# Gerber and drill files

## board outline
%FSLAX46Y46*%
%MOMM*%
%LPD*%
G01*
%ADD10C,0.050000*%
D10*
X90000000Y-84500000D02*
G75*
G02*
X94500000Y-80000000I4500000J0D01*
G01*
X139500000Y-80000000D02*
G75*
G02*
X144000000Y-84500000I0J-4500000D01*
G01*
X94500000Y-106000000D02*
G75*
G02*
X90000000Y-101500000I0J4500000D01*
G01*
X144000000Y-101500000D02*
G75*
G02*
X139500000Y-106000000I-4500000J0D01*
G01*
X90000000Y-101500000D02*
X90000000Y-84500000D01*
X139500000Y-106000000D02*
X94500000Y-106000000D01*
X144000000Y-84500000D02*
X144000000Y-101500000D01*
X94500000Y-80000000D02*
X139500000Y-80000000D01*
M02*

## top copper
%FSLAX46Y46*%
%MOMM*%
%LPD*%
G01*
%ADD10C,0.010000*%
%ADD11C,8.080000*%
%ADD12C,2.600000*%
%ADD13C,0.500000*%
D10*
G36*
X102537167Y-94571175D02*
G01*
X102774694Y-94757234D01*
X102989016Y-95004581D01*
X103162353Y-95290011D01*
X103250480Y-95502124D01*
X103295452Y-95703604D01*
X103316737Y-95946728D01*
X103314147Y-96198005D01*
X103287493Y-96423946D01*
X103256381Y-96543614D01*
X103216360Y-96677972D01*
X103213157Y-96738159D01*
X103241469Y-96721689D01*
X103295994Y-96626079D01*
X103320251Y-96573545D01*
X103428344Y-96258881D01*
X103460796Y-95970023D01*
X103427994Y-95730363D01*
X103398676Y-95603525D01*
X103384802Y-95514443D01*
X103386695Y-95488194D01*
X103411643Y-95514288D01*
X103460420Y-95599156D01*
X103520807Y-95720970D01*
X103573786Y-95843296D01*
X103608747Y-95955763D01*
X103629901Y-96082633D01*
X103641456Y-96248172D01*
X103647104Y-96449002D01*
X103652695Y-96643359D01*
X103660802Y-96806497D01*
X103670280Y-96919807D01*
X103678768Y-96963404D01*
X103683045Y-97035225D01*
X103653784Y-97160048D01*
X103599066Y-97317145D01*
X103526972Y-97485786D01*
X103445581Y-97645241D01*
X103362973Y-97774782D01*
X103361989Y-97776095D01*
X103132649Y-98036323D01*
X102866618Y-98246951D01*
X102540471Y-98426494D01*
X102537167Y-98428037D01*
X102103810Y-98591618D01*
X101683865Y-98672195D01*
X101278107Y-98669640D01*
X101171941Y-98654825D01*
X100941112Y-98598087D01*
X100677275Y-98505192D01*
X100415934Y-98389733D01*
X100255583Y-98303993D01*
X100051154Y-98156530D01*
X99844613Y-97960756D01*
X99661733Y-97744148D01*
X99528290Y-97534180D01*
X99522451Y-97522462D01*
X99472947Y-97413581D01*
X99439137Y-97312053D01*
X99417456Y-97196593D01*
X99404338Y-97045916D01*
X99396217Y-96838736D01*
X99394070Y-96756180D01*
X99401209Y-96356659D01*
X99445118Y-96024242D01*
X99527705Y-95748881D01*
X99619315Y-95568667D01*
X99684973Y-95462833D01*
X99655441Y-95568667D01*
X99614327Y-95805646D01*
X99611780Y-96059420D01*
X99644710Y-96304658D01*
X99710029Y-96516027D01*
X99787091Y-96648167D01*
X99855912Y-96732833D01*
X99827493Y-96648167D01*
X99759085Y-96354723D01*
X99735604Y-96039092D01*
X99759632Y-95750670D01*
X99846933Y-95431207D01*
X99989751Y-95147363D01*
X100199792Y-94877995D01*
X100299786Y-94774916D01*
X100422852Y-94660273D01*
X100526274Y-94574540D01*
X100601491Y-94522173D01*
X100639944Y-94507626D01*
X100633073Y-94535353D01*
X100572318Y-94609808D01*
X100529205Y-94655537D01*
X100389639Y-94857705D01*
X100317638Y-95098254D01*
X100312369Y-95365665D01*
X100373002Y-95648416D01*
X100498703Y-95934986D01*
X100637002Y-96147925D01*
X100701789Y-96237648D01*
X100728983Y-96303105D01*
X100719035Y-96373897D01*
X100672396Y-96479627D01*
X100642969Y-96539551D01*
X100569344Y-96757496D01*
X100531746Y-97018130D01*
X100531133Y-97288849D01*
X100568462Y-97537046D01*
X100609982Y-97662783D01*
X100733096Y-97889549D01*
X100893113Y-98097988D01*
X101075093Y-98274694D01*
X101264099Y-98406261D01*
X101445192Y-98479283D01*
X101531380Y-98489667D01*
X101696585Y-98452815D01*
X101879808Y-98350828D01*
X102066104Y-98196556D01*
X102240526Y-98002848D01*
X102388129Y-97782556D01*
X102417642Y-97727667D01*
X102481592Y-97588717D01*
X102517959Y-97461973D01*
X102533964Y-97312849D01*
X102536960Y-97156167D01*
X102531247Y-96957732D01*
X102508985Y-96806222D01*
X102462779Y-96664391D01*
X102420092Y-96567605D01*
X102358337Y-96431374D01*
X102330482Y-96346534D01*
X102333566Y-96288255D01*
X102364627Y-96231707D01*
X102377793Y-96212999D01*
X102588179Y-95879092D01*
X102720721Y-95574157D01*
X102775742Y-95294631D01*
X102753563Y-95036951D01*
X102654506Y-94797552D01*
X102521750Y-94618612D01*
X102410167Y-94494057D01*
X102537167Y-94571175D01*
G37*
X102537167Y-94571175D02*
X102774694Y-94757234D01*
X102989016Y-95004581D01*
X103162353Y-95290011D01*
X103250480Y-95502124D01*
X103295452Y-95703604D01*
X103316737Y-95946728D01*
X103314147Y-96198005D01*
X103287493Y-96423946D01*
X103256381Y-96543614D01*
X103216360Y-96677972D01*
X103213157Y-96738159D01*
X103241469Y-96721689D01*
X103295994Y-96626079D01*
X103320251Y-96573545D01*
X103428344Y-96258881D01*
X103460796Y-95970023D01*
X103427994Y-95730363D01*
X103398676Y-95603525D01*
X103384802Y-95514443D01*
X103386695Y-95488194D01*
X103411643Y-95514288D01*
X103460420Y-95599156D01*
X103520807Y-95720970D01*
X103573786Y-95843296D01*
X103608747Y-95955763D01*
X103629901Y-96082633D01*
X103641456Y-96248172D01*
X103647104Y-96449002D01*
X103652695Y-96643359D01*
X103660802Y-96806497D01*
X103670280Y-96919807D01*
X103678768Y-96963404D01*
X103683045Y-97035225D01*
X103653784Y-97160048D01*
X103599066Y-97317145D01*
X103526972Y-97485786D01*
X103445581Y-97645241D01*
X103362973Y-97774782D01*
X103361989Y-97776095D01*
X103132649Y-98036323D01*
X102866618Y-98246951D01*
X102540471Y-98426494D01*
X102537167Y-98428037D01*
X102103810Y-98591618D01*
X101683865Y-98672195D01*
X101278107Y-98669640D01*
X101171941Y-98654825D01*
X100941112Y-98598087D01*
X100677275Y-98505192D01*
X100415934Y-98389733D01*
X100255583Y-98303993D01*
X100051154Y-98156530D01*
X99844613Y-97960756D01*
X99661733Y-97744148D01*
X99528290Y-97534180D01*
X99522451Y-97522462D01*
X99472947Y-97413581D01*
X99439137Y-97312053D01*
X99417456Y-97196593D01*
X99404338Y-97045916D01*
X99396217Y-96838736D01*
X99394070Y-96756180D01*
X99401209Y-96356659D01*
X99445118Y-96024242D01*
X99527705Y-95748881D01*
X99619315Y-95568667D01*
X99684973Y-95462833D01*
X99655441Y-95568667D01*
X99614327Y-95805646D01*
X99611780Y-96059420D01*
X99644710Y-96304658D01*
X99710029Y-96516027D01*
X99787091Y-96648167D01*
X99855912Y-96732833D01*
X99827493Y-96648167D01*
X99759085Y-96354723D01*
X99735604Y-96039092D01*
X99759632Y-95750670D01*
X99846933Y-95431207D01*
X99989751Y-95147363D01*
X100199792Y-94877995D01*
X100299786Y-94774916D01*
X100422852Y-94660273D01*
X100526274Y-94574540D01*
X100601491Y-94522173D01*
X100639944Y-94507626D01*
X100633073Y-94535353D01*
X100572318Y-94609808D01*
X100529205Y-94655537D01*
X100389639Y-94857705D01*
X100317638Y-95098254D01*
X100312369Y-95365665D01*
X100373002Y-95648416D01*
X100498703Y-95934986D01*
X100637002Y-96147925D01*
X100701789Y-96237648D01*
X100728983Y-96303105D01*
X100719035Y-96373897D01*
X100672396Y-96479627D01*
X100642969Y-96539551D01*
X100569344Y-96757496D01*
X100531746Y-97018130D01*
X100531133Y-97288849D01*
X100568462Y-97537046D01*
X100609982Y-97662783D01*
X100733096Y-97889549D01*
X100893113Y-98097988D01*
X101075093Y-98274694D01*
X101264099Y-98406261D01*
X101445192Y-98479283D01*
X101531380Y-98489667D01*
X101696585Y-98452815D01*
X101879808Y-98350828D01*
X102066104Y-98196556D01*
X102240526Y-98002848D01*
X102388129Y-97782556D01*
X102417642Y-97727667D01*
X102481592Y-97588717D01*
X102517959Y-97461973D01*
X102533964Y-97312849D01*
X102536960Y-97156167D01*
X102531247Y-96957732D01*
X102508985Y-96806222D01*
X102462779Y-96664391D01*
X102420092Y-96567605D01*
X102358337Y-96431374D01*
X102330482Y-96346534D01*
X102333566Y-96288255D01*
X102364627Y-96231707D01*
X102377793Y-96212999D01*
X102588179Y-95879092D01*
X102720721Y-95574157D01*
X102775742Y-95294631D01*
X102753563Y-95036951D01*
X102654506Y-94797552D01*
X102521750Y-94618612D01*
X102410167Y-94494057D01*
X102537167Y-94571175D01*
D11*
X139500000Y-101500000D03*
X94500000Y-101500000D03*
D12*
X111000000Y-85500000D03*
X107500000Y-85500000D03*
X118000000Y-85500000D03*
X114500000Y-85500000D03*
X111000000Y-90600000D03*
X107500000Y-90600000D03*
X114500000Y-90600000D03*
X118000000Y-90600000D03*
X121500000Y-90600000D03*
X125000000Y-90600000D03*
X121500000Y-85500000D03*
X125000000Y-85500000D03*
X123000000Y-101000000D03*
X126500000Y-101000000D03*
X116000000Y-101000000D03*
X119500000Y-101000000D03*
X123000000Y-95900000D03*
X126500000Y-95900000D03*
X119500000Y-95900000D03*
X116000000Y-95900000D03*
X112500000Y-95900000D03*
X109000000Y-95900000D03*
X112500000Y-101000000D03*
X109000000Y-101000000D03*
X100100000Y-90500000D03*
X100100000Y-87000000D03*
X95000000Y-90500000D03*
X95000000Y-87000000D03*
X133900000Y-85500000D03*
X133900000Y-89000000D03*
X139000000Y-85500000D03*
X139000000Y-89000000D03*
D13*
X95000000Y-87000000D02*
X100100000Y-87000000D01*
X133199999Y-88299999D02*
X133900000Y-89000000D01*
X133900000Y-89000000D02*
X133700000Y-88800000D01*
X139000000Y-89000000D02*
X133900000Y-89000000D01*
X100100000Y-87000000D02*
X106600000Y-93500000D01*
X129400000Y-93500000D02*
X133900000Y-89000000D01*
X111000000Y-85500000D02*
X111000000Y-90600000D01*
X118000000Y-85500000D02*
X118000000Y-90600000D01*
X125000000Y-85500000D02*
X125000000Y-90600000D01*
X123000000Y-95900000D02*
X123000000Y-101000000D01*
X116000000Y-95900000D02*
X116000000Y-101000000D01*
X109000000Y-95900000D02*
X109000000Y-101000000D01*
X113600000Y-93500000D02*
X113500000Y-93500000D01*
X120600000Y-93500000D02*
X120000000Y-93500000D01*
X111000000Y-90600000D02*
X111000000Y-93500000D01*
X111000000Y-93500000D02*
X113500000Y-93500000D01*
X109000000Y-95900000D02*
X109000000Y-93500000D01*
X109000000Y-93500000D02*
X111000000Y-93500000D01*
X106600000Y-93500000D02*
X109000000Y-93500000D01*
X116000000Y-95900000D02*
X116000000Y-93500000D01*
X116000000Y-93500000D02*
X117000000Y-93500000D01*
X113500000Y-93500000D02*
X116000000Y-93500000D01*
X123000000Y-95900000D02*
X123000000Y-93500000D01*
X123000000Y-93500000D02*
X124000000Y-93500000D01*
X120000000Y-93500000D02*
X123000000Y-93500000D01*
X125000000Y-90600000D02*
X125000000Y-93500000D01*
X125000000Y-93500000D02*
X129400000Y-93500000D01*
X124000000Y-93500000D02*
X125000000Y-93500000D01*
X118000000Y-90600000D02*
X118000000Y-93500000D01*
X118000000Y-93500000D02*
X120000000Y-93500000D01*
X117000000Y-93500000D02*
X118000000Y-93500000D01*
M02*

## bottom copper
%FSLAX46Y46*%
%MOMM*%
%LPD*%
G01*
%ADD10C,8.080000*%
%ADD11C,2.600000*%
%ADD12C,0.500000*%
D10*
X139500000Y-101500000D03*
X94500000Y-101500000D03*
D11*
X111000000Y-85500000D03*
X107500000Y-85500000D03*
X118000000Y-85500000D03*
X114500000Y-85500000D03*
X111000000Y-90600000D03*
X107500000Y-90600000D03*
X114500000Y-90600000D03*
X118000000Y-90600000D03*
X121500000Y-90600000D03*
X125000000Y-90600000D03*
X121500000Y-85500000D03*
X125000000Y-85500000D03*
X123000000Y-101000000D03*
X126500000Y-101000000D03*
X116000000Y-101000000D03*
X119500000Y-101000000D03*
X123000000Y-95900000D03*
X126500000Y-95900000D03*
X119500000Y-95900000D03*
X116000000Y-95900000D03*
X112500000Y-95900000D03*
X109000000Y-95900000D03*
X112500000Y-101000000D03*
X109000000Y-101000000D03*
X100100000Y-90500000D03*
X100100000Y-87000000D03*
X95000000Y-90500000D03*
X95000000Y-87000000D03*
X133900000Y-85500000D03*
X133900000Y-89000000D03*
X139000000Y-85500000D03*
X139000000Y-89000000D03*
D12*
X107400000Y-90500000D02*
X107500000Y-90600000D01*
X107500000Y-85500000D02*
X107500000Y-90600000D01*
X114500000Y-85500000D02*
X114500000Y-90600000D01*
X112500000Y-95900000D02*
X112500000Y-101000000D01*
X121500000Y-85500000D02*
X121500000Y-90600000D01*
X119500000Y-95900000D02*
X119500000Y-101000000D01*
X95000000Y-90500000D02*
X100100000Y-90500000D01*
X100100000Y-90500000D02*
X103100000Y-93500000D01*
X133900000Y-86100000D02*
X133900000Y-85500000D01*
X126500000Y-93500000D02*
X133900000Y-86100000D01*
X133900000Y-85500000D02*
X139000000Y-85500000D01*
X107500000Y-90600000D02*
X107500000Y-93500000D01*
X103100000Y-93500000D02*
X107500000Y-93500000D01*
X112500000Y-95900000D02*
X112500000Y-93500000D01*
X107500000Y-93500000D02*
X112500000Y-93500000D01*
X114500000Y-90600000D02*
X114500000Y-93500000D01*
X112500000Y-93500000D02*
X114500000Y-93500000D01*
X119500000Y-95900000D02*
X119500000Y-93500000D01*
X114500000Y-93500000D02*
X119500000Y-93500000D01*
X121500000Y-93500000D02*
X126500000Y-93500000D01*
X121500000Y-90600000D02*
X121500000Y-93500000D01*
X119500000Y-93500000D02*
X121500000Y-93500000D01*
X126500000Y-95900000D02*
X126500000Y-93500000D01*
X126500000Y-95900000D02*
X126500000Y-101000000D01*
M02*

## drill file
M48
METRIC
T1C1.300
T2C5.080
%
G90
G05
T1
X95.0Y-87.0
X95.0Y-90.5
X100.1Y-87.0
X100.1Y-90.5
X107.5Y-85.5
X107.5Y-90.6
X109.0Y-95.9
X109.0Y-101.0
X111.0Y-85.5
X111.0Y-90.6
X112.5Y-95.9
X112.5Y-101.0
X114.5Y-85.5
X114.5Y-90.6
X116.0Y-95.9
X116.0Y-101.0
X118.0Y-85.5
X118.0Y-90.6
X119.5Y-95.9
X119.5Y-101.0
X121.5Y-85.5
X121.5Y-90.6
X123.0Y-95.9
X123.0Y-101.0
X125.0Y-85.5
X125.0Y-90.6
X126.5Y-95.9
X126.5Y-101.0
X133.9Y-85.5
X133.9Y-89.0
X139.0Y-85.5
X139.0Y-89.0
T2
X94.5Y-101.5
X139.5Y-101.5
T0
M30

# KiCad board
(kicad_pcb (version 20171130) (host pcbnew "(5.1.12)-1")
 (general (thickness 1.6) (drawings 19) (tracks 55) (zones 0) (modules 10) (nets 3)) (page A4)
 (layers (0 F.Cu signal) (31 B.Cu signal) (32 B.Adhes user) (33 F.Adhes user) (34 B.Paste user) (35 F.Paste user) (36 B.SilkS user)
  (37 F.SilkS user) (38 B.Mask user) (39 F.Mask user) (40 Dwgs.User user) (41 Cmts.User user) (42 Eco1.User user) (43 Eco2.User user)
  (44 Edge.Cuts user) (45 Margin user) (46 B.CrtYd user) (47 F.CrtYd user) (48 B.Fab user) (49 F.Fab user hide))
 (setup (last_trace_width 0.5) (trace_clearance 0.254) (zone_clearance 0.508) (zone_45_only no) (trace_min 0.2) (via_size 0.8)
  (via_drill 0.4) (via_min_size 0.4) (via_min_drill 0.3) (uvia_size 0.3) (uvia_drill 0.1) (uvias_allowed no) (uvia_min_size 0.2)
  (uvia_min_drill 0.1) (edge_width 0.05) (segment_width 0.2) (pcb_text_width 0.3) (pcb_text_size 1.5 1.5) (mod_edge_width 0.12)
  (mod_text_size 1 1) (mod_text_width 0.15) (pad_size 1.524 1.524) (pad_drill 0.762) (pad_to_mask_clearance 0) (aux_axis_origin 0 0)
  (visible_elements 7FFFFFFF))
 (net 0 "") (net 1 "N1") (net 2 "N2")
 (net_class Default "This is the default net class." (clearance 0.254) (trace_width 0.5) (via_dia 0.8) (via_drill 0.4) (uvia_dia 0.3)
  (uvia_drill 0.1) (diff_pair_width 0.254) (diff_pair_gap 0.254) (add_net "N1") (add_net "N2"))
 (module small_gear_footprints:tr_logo (layer F.Cu) (at 132 96.5)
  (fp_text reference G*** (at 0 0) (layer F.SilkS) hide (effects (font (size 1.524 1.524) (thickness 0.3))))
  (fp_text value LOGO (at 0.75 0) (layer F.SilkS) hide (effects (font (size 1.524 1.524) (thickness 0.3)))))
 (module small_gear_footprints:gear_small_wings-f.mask (layer F.Cu) (at 101.5 96.5)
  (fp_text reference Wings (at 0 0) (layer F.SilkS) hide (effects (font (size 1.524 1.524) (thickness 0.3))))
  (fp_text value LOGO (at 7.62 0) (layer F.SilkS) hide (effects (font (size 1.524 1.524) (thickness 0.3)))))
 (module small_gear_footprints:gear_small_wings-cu (layer F.Cu) (at 101.5 96.5)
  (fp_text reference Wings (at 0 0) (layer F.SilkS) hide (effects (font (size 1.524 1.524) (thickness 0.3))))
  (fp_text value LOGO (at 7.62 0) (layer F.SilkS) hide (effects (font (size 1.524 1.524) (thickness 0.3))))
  (fp_poly
   (pts (xy 1.037167 -1.928825) (xy 1.274694 -1.742766) (xy 1.489016 -1.495419) (xy 1.662353 -1.209989) (xy 1.75048 -0.997876)
    (xy 1.795452 -0.796396) (xy 1.816737 -0.553272) (xy 1.814147 -0.301995) (xy 1.787493 -0.076054) (xy 1.756381 0.043614)
    (xy 1.71636 0.177972) (xy 1.713157 0.238159) (xy 1.741469 0.221689) (xy 1.795994 0.126079) (xy 1.820251 0.073545)
    (xy 1.928344 -0.241119) (xy 1.960796 -0.529977) (xy 1.927994 -0.769637) (xy 1.898676 -0.896475) (xy 1.884802 -0.985557)
    (xy 1.886695 -1.011806) (xy 1.911643 -0.985712) (xy 1.96042 -0.900844) (xy 2.020807 -0.77903) (xy 2.073786 -0.656704)
    (xy 2.108747 -0.544237) (xy 2.129901 -0.417367) (xy 2.141456 -0.251828) (xy 2.147104 -0.050998) (xy 2.152695 0.143359)
    (xy 2.160802 0.306497) (xy 2.17028 0.419807) (xy 2.178768 0.463404) (xy 2.183045 0.535225) (xy 2.153784 0.660048) (xy 2.099066 0.817145)
    (xy 2.026972 0.985786) (xy 1.945581 1.145241) (xy 1.862973 1.274782) (xy 1.861989 1.276095) (xy 1.632649 1.536323)
    (xy 1.366618 1.746951) (xy 1.040471 1.926494) (xy 1.037167 1.928037) (xy 0.60381 2.091618) (xy 0.183865 2.172195) (xy -0.221893 2.16964)
    (xy -0.328059 2.154825) (xy -0.558888 2.098087) (xy -0.822725 2.005192) (xy -1.084066 1.889733) (xy -1.244417 1.803993)
    (xy -1.448846 1.65653) (xy -1.655387 1.460756) (xy -1.838267 1.244148) (xy -1.97171 1.03418) (xy -1.977549 1.022462)
    (xy -2.027053 0.913581) (xy -2.060863 0.812053) (xy -2.082544 0.696593) (xy -2.095662 0.545916) (xy -2.103783 0.338736)
    (xy -2.10593 0.25618) (xy -2.098791 -0.143341) (xy -2.054882 -0.475758) (xy -1.972295 -0.751119) (xy -1.880685 -0.931333)
    (xy -1.815027 -1.037167) (xy -1.844559 -0.931333) (xy -1.885673 -0.694354) (xy -1.88822 -0.44058) (xy -1.85529 -0.195342)
    (xy -1.789971 0.016027) (xy -1.712909 0.148167) (xy -1.644088 0.232833) (xy -1.672507 0.148167) (xy -1.740915 -0.145277)
    (xy -1.764396 -0.460908) (xy -1.740368 -0.74933) (xy -1.653067 -1.068793) (xy -1.510249 -1.352637) (xy -1.300208 -1.622005)
    (xy -1.200214 -1.725084) (xy -1.077148 -1.839727) (xy -0.973726 -1.92546) (xy -0.898509 -1.977827) (xy -0.860056 -1.992374)
    (xy -0.866927 -1.964647) (xy -0.927682 -1.890192) (xy -0.970795 -1.844463) (xy -1.110361 -1.642295) (xy -1.182362 -1.401746)
    (xy -1.187631 -1.134335) (xy -1.126998 -0.851584) (xy -1.001297 -0.565014) (xy -0.862998 -0.352075) (xy -0.798211 -0.262352)
    (xy -0.771017 -0.196895) (xy -0.780965 -0.126103) (xy -0.827604 -0.020373) (xy -0.857031 0.039551) (xy -0.930656 0.257496)
    (xy -0.968254 0.51813) (xy -0.968867 0.788849) (xy -0.931538 1.037046) (xy -0.890018 1.162783) (xy -0.766904 1.389549)
    (xy -0.606887 1.597988) (xy -0.424907 1.774694) (xy -0.235901 1.906261) (xy -0.054808 1.979283) (xy 0.03138 1.989667)
    (xy 0.196585 1.952815) (xy 0.379808 1.850828) (xy 0.566104 1.696556) (xy 0.740526 1.502848) (xy 0.888129 1.282556)
    (xy 0.917642 1.227667) (xy 0.981592 1.088717) (xy 1.017959 0.961973) (xy 1.033964 0.812849) (xy 1.03696 0.656167) (xy 1.031247 0.457732)
    (xy 1.008985 0.306222) (xy 0.962779 0.164391) (xy 0.920092 0.067605) (xy 0.858337 -0.068626) (xy 0.830482 -0.153466)
    (xy 0.833566 -0.211745) (xy 0.864627 -0.268293) (xy 0.877793 -0.287001) (xy 1.088179 -0.620908) (xy 1.220721 -0.925843)
    (xy 1.275742 -1.205369) (xy 1.253563 -1.463049) (xy 1.154506 -1.702448) (xy 1.02175 -1.881388) (xy 0.910167 -2.005943)
    (xy 1.037167 -1.928825))
   (layer F.Cu) (width 0.01)))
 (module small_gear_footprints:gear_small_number (layer F.Cu) (at 101.5 96.5)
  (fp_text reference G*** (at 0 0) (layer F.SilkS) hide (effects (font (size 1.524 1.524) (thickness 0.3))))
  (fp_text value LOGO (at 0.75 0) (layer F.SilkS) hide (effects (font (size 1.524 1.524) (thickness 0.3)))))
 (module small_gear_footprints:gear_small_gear (layer F.Cu) (at 101.5 96.5)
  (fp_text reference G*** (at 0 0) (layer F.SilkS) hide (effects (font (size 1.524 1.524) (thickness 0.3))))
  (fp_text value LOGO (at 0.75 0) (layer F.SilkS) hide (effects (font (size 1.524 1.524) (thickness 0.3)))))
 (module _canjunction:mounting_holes (layer F.Cu) (at 94.5 101.5)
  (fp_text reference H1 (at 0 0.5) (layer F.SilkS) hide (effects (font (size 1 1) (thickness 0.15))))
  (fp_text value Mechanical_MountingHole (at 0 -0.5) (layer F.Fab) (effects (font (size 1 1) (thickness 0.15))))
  (pad "" thru_hole circle (at 45 0) (size 8.08 8.08) (drill 5.08) (layers *.Cu *.Mask))
  (pad "" thru_hole circle (at 0 0) (size 8.08 8.08) (drill 5.08) (layers *.Cu *.Mask)))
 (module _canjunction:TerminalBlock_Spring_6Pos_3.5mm (layer F.Cu) (at 125 85.5 180)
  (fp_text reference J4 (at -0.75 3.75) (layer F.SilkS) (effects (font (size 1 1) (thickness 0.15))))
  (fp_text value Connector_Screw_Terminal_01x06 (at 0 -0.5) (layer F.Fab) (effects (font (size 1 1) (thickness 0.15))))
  (pad 5 thru_hole circle (at 14 0 180) (size 2.6 2.6) (drill 1.3) (layers *.Cu *.Mask) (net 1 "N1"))
  (pad 6 thru_hole circle (at 17.5 0 180) (size 2.6 2.6) (drill 1.3) (layers *.Cu *.Mask) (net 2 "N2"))
  (pad 3 thru_hole circle (at 7 0 180) (size 2.6 2.6) (drill 1.3) (layers *.Cu *.Mask) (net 1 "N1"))
  (pad 4 thru_hole circle (at 10.5 0 180) (size 2.6 2.6) (drill 1.3) (layers *.Cu *.Mask) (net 2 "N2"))
  (pad 5 thru_hole circle (at 14 -5.1 180) (size 2.6 2.6) (drill 1.3) (layers *.Cu *.Mask) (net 1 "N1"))
  (pad 6 thru_hole circle (at 17.5 -5.1 180) (size 2.6 2.6) (drill 1.3) (layers *.Cu *.Mask) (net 2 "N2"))
  (pad 4 thru_hole circle (at 10.5 -5.1 180) (size 2.6 2.6) (drill 1.3) (layers *.Cu *.Mask) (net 2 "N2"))
  (pad 3 thru_hole circle (at 7 -5.1 180) (size 2.6 2.6) (drill 1.3) (layers *.Cu *.Mask) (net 1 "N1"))
  (pad 2 thru_hole circle (at 3.5 -5.1 180) (size 2.6 2.6) (drill 1.3) (layers *.Cu *.Mask) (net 2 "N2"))
  (pad 1 thru_hole circle (at 0 -5.1 180) (size 2.6 2.6) (drill 1.3) (layers *.Cu *.Mask) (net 1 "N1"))
  (pad 2 thru_hole circle (at 3.5 0 180) (size 2.6 2.6) (drill 1.3) (layers *.Cu *.Mask) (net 2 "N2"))
  (pad 1 thru_hole circle (at 0 0 180) (size 2.6 2.6) (drill 1.3) (layers *.Cu *.Mask) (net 1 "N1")))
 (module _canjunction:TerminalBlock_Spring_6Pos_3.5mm (layer F.Cu) (at 109 101)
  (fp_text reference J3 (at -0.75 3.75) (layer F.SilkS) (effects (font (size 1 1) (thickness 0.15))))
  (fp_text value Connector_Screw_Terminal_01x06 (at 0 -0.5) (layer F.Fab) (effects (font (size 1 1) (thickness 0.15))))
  (pad 5 thru_hole circle (at 14 0) (size 2.6 2.6) (drill 1.3) (layers *.Cu *.Mask) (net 1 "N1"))
  (pad 6 thru_hole circle (at 17.5 0) (size 2.6 2.6) (drill 1.3) (layers *.Cu *.Mask) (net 2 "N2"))
  (pad 3 thru_hole circle (at 7 0) (size 2.6 2.6) (drill 1.3) (layers *.Cu *.Mask) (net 1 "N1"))
  (pad 4 thru_hole circle (at 10.5 0) (size 2.6 2.6) (drill 1.3) (layers *.Cu *.Mask) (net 2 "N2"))
  (pad 5 thru_hole circle (at 14 -5.1) (size 2.6 2.6) (drill 1.3) (layers *.Cu *.Mask) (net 1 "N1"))
  (pad 6 thru_hole circle (at 17.5 -5.1) (size 2.6 2.6) (drill 1.3) (layers *.Cu *.Mask) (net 2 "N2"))
  (pad 4 thru_hole circle (at 10.5 -5.1) (size 2.6 2.6) (drill 1.3) (layers *.Cu *.Mask) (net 2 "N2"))
  (pad 3 thru_hole circle (at 7 -5.1) (size 2.6 2.6) (drill 1.3) (layers *.Cu *.Mask) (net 1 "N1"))
  (pad 2 thru_hole circle (at 3.5 -5.1) (size 2.6 2.6) (drill 1.3) (layers *.Cu *.Mask) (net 2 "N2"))
  (pad 1 thru_hole circle (at 0 -5.1) (size 2.6 2.6) (drill 1.3) (layers *.Cu *.Mask) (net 1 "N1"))
  (pad 2 thru_hole circle (at 3.5 0) (size 2.6 2.6) (drill 1.3) (layers *.Cu *.Mask) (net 2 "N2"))
  (pad 1 thru_hole circle (at 0 0) (size 2.6 2.6) (drill 1.3) (layers *.Cu *.Mask) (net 1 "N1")))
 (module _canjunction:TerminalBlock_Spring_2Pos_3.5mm (layer F.Cu) (at 95 87 270)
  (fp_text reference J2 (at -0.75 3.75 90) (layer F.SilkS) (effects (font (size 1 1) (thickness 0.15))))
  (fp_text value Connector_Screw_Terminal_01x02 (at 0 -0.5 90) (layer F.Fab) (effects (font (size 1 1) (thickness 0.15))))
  (pad 2 thru_hole circle (at 3.5 -5.1 270) (size 2.6 2.6) (drill 1.3) (layers *.Cu *.Mask) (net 2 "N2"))
  (pad 1 thru_hole circle (at 0 -5.1 270) (size 2.6 2.6) (drill 1.3) (layers *.Cu *.Mask) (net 1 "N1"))
  (pad 2 thru_hole circle (at 3.5 0 270) (size 2.6 2.6) (drill 1.3) (layers *.Cu *.Mask) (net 2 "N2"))
  (pad 1 thru_hole circle (at 0 0 270) (size 2.6 2.6) (drill 1.3) (layers *.Cu *.Mask) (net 1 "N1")))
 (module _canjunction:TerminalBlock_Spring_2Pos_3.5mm (layer F.Cu) (at 139 89 90)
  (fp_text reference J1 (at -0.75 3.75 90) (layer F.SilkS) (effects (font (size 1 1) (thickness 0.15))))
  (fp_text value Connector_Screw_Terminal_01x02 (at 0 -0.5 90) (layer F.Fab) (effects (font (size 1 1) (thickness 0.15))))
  (pad 2 thru_hole circle (at 3.5 -5.1 90) (size 2.6 2.6) (drill 1.3) (layers *.Cu *.Mask) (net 2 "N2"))
  (pad 1 thru_hole circle (at 0 -5.1 90) (size 2.6 2.6) (drill 1.3) (layers *.Cu *.Mask) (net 1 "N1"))
  (pad 2 thru_hole circle (at 3.5 0 90) (size 2.6 2.6) (drill 1.3) (layers *.Cu *.Mask) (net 2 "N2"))
  (pad 1 thru_hole circle (at 0 0 90) (size 2.6 2.6) (drill 1.3) (layers *.Cu *.Mask) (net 1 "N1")))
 (gr_arc (start 94.5 84.5) (end 94.5 80) (angle -90) (layer Edge.Cuts) (width 0.05))
 (gr_arc (start 139.5 84.5) (end 144 84.5) (angle -90) (layer Edge.Cuts) (width 0.05))
 (gr_arc (start 94.5 101.5) (end 90 101.5) (angle -90) (layer Edge.Cuts) (width 0.05))
 (gr_arc (start 139.5 101.5) (end 139.5 106) (angle -90) (layer Edge.Cuts) (width 0.05))
 (gr_line (start 90 101.5) (end 90 84.5) (layer Edge.Cuts) (width 0.05))
 (gr_line (start 139.5 106) (end 94.5 106) (layer Edge.Cuts) (width 0.05))
 (gr_line (start 144 84.5) (end 144 101.5) (layer Edge.Cuts) (width 0.05))
 (gr_line (start 94.5 80) (end 139.5 80) (layer Edge.Cuts) (width 0.05))
 (segment (start 107.4 90.5) (end 107.5 90.6) (width 0.5) (layer B.Cu) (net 2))
 (segment (start 107.5 85.5) (end 107.5 90.6) (width 0.5) (layer B.Cu) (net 2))
 (segment (start 114.5 85.5) (end 114.5 90.6) (width 0.5) (layer B.Cu) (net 2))
 (segment (start 112.5 95.9) (end 112.5 101) (width 0.5) (layer B.Cu) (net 2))
 (segment (start 121.5 85.5) (end 121.5 90.6) (width 0.5) (layer B.Cu) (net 2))
 (segment (start 119.5 95.9) (end 119.5 101) (width 0.5) (layer B.Cu) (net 2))
 (segment (start 95 90.5) (end 100.1 90.5) (width 0.5) (layer B.Cu) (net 2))
 (segment (start 100.1 90.5) (end 103.1 93.5) (width 0.5) (layer B.Cu) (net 2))
 (segment (start 133.9 86.1) (end 133.9 85.5) (width 0.5) (layer B.Cu) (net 2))
 (segment (start 126.5 93.5) (end 133.9 86.1) (width 0.5) (layer B.Cu) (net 2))
 (segment (start 133.9 85.5) (end 139 85.5) (width 0.5) (layer B.Cu) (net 2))
 (segment (start 107.5 90.6) (end 107.5 93.5) (width 0.5) (layer B.Cu) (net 2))
 (segment (start 103.1 93.5) (end 107.5 93.5) (width 0.5) (layer B.Cu) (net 2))
 (segment (start 112.5 95.9) (end 112.5 93.5) (width 0.5) (layer B.Cu) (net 2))
 (segment (start 107.5 93.5) (end 112.5 93.5) (width 0.5) (layer B.Cu) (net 2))
 (segment (start 114.5 90.6) (end 114.5 93.5) (width 0.5) (layer B.Cu) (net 2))
 (segment (start 112.5 93.5) (end 114.5 93.5) (width 0.5) (layer B.Cu) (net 2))
 (segment (start 119.5 95.9) (end 119.5 93.5) (width 0.5) (layer B.Cu) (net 2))
 (segment (start 114.5 93.5) (end 119.5 93.5) (width 0.5) (layer B.Cu) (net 2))
 (segment (start 121.5 93.5) (end 126.5 93.5) (width 0.5) (layer B.Cu) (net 2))
 (segment (start 121.5 90.6) (end 121.5 93.5) (width 0.5) (layer B.Cu) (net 2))
 (segment (start 119.5 93.5) (end 121.5 93.5) (width 0.5) (layer B.Cu) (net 2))
 (segment (start 126.5 95.9) (end 126.5 93.5) (width 0.5) (layer B.Cu) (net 2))
 (segment (start 126.5 95.9) (end 126.5 101) (width 0.5) (layer B.Cu) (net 2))
 (segment (start 95 87) (end 100.1 87) (width 0.5) (layer F.Cu) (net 1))
 (segment (start 133.199999 88.299999) (end 133.9 89) (width 0.5) (layer F.Cu) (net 1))
 (segment (start 133.9 89) (end 133.7 88.8) (width 0.5) (layer F.Cu) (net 1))
 (segment (start 139 89) (end 133.9 89) (width 0.5) (layer F.Cu) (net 1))
 (segment (start 100.1 87) (end 106.6 93.5) (width 0.5) (layer F.Cu) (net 1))
 (segment (start 129.4 93.5) (end 133.9 89) (width 0.5) (layer F.Cu) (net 1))
 (segment (start 111 85.5) (end 111 90.6) (width 0.5) (layer F.Cu) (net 1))
 (segment (start 118 85.5) (end 118 90.6) (width 0.5) (layer F.Cu) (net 1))
 (segment (start 125 85.5) (end 125 90.6) (width 0.5) (layer F.Cu) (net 1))
 (segment (start 123 95.9) (end 123 101) (width 0.5) (layer F.Cu) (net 1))
 (segment (start 116 95.9) (end 116 101) (width 0.5) (layer F.Cu) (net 1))
 (segment (start 109 95.9) (end 109 101) (width 0.5) (layer F.Cu) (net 1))
 (segment (start 113.6 93.5) (end 113.5 93.5) (width 0.5) (layer F.Cu) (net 1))
 (segment (start 120.6 93.5) (end 120 93.5) (width 0.5) (layer F.Cu) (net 1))
 (segment (start 111 90.6) (end 111 93.5) (width 0.5) (layer F.Cu) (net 1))
 (segment (start 111 93.5) (end 113.5 93.5) (width 0.5) (layer F.Cu) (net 1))
 (segment (start 109 95.9) (end 109 93.5) (width 0.5) (layer F.Cu) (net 1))
 (segment (start 109 93.5) (end 111 93.5) (width 0.5) (layer F.Cu) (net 1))
 (segment (start 106.6 93.5) (end 109 93.5) (width 0.5) (layer F.Cu) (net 1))
 (segment (start 116 95.9) (end 116 93.5) (width 0.5) (layer F.Cu) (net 1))
 (segment (start 116 93.5) (end 117 93.5) (width 0.5) (layer F.Cu) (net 1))
 (segment (start 113.5 93.5) (end 116 93.5) (width 0.5) (layer F.Cu) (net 1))
 (segment (start 123 95.9) (end 123 93.5) (width 0.5) (layer F.Cu) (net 1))
 (segment (start 123 93.5) (end 124 93.5) (width 0.5) (layer F.Cu) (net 1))
 (segment (start 120 93.5) (end 123 93.5) (width 0.5) (layer F.Cu) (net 1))
 (segment (start 125 90.6) (end 125 93.5) (width 0.5) (layer F.Cu) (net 1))
 (segment (start 125 93.5) (end 129.4 93.5) (width 0.5) (layer F.Cu) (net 1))
 (segment (start 124 93.5) (end 125 93.5) (width 0.5) (layer F.Cu) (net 1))
 (segment (start 118 90.6) (end 118 93.5) (width 0.5) (layer F.Cu) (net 1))
 (segment (start 118 93.5) (end 120 93.5) (width 0.5) (layer F.Cu) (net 1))
 (segment (start 117 93.5) (end 118 93.5) (width 0.5) (layer F.Cu) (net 1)))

